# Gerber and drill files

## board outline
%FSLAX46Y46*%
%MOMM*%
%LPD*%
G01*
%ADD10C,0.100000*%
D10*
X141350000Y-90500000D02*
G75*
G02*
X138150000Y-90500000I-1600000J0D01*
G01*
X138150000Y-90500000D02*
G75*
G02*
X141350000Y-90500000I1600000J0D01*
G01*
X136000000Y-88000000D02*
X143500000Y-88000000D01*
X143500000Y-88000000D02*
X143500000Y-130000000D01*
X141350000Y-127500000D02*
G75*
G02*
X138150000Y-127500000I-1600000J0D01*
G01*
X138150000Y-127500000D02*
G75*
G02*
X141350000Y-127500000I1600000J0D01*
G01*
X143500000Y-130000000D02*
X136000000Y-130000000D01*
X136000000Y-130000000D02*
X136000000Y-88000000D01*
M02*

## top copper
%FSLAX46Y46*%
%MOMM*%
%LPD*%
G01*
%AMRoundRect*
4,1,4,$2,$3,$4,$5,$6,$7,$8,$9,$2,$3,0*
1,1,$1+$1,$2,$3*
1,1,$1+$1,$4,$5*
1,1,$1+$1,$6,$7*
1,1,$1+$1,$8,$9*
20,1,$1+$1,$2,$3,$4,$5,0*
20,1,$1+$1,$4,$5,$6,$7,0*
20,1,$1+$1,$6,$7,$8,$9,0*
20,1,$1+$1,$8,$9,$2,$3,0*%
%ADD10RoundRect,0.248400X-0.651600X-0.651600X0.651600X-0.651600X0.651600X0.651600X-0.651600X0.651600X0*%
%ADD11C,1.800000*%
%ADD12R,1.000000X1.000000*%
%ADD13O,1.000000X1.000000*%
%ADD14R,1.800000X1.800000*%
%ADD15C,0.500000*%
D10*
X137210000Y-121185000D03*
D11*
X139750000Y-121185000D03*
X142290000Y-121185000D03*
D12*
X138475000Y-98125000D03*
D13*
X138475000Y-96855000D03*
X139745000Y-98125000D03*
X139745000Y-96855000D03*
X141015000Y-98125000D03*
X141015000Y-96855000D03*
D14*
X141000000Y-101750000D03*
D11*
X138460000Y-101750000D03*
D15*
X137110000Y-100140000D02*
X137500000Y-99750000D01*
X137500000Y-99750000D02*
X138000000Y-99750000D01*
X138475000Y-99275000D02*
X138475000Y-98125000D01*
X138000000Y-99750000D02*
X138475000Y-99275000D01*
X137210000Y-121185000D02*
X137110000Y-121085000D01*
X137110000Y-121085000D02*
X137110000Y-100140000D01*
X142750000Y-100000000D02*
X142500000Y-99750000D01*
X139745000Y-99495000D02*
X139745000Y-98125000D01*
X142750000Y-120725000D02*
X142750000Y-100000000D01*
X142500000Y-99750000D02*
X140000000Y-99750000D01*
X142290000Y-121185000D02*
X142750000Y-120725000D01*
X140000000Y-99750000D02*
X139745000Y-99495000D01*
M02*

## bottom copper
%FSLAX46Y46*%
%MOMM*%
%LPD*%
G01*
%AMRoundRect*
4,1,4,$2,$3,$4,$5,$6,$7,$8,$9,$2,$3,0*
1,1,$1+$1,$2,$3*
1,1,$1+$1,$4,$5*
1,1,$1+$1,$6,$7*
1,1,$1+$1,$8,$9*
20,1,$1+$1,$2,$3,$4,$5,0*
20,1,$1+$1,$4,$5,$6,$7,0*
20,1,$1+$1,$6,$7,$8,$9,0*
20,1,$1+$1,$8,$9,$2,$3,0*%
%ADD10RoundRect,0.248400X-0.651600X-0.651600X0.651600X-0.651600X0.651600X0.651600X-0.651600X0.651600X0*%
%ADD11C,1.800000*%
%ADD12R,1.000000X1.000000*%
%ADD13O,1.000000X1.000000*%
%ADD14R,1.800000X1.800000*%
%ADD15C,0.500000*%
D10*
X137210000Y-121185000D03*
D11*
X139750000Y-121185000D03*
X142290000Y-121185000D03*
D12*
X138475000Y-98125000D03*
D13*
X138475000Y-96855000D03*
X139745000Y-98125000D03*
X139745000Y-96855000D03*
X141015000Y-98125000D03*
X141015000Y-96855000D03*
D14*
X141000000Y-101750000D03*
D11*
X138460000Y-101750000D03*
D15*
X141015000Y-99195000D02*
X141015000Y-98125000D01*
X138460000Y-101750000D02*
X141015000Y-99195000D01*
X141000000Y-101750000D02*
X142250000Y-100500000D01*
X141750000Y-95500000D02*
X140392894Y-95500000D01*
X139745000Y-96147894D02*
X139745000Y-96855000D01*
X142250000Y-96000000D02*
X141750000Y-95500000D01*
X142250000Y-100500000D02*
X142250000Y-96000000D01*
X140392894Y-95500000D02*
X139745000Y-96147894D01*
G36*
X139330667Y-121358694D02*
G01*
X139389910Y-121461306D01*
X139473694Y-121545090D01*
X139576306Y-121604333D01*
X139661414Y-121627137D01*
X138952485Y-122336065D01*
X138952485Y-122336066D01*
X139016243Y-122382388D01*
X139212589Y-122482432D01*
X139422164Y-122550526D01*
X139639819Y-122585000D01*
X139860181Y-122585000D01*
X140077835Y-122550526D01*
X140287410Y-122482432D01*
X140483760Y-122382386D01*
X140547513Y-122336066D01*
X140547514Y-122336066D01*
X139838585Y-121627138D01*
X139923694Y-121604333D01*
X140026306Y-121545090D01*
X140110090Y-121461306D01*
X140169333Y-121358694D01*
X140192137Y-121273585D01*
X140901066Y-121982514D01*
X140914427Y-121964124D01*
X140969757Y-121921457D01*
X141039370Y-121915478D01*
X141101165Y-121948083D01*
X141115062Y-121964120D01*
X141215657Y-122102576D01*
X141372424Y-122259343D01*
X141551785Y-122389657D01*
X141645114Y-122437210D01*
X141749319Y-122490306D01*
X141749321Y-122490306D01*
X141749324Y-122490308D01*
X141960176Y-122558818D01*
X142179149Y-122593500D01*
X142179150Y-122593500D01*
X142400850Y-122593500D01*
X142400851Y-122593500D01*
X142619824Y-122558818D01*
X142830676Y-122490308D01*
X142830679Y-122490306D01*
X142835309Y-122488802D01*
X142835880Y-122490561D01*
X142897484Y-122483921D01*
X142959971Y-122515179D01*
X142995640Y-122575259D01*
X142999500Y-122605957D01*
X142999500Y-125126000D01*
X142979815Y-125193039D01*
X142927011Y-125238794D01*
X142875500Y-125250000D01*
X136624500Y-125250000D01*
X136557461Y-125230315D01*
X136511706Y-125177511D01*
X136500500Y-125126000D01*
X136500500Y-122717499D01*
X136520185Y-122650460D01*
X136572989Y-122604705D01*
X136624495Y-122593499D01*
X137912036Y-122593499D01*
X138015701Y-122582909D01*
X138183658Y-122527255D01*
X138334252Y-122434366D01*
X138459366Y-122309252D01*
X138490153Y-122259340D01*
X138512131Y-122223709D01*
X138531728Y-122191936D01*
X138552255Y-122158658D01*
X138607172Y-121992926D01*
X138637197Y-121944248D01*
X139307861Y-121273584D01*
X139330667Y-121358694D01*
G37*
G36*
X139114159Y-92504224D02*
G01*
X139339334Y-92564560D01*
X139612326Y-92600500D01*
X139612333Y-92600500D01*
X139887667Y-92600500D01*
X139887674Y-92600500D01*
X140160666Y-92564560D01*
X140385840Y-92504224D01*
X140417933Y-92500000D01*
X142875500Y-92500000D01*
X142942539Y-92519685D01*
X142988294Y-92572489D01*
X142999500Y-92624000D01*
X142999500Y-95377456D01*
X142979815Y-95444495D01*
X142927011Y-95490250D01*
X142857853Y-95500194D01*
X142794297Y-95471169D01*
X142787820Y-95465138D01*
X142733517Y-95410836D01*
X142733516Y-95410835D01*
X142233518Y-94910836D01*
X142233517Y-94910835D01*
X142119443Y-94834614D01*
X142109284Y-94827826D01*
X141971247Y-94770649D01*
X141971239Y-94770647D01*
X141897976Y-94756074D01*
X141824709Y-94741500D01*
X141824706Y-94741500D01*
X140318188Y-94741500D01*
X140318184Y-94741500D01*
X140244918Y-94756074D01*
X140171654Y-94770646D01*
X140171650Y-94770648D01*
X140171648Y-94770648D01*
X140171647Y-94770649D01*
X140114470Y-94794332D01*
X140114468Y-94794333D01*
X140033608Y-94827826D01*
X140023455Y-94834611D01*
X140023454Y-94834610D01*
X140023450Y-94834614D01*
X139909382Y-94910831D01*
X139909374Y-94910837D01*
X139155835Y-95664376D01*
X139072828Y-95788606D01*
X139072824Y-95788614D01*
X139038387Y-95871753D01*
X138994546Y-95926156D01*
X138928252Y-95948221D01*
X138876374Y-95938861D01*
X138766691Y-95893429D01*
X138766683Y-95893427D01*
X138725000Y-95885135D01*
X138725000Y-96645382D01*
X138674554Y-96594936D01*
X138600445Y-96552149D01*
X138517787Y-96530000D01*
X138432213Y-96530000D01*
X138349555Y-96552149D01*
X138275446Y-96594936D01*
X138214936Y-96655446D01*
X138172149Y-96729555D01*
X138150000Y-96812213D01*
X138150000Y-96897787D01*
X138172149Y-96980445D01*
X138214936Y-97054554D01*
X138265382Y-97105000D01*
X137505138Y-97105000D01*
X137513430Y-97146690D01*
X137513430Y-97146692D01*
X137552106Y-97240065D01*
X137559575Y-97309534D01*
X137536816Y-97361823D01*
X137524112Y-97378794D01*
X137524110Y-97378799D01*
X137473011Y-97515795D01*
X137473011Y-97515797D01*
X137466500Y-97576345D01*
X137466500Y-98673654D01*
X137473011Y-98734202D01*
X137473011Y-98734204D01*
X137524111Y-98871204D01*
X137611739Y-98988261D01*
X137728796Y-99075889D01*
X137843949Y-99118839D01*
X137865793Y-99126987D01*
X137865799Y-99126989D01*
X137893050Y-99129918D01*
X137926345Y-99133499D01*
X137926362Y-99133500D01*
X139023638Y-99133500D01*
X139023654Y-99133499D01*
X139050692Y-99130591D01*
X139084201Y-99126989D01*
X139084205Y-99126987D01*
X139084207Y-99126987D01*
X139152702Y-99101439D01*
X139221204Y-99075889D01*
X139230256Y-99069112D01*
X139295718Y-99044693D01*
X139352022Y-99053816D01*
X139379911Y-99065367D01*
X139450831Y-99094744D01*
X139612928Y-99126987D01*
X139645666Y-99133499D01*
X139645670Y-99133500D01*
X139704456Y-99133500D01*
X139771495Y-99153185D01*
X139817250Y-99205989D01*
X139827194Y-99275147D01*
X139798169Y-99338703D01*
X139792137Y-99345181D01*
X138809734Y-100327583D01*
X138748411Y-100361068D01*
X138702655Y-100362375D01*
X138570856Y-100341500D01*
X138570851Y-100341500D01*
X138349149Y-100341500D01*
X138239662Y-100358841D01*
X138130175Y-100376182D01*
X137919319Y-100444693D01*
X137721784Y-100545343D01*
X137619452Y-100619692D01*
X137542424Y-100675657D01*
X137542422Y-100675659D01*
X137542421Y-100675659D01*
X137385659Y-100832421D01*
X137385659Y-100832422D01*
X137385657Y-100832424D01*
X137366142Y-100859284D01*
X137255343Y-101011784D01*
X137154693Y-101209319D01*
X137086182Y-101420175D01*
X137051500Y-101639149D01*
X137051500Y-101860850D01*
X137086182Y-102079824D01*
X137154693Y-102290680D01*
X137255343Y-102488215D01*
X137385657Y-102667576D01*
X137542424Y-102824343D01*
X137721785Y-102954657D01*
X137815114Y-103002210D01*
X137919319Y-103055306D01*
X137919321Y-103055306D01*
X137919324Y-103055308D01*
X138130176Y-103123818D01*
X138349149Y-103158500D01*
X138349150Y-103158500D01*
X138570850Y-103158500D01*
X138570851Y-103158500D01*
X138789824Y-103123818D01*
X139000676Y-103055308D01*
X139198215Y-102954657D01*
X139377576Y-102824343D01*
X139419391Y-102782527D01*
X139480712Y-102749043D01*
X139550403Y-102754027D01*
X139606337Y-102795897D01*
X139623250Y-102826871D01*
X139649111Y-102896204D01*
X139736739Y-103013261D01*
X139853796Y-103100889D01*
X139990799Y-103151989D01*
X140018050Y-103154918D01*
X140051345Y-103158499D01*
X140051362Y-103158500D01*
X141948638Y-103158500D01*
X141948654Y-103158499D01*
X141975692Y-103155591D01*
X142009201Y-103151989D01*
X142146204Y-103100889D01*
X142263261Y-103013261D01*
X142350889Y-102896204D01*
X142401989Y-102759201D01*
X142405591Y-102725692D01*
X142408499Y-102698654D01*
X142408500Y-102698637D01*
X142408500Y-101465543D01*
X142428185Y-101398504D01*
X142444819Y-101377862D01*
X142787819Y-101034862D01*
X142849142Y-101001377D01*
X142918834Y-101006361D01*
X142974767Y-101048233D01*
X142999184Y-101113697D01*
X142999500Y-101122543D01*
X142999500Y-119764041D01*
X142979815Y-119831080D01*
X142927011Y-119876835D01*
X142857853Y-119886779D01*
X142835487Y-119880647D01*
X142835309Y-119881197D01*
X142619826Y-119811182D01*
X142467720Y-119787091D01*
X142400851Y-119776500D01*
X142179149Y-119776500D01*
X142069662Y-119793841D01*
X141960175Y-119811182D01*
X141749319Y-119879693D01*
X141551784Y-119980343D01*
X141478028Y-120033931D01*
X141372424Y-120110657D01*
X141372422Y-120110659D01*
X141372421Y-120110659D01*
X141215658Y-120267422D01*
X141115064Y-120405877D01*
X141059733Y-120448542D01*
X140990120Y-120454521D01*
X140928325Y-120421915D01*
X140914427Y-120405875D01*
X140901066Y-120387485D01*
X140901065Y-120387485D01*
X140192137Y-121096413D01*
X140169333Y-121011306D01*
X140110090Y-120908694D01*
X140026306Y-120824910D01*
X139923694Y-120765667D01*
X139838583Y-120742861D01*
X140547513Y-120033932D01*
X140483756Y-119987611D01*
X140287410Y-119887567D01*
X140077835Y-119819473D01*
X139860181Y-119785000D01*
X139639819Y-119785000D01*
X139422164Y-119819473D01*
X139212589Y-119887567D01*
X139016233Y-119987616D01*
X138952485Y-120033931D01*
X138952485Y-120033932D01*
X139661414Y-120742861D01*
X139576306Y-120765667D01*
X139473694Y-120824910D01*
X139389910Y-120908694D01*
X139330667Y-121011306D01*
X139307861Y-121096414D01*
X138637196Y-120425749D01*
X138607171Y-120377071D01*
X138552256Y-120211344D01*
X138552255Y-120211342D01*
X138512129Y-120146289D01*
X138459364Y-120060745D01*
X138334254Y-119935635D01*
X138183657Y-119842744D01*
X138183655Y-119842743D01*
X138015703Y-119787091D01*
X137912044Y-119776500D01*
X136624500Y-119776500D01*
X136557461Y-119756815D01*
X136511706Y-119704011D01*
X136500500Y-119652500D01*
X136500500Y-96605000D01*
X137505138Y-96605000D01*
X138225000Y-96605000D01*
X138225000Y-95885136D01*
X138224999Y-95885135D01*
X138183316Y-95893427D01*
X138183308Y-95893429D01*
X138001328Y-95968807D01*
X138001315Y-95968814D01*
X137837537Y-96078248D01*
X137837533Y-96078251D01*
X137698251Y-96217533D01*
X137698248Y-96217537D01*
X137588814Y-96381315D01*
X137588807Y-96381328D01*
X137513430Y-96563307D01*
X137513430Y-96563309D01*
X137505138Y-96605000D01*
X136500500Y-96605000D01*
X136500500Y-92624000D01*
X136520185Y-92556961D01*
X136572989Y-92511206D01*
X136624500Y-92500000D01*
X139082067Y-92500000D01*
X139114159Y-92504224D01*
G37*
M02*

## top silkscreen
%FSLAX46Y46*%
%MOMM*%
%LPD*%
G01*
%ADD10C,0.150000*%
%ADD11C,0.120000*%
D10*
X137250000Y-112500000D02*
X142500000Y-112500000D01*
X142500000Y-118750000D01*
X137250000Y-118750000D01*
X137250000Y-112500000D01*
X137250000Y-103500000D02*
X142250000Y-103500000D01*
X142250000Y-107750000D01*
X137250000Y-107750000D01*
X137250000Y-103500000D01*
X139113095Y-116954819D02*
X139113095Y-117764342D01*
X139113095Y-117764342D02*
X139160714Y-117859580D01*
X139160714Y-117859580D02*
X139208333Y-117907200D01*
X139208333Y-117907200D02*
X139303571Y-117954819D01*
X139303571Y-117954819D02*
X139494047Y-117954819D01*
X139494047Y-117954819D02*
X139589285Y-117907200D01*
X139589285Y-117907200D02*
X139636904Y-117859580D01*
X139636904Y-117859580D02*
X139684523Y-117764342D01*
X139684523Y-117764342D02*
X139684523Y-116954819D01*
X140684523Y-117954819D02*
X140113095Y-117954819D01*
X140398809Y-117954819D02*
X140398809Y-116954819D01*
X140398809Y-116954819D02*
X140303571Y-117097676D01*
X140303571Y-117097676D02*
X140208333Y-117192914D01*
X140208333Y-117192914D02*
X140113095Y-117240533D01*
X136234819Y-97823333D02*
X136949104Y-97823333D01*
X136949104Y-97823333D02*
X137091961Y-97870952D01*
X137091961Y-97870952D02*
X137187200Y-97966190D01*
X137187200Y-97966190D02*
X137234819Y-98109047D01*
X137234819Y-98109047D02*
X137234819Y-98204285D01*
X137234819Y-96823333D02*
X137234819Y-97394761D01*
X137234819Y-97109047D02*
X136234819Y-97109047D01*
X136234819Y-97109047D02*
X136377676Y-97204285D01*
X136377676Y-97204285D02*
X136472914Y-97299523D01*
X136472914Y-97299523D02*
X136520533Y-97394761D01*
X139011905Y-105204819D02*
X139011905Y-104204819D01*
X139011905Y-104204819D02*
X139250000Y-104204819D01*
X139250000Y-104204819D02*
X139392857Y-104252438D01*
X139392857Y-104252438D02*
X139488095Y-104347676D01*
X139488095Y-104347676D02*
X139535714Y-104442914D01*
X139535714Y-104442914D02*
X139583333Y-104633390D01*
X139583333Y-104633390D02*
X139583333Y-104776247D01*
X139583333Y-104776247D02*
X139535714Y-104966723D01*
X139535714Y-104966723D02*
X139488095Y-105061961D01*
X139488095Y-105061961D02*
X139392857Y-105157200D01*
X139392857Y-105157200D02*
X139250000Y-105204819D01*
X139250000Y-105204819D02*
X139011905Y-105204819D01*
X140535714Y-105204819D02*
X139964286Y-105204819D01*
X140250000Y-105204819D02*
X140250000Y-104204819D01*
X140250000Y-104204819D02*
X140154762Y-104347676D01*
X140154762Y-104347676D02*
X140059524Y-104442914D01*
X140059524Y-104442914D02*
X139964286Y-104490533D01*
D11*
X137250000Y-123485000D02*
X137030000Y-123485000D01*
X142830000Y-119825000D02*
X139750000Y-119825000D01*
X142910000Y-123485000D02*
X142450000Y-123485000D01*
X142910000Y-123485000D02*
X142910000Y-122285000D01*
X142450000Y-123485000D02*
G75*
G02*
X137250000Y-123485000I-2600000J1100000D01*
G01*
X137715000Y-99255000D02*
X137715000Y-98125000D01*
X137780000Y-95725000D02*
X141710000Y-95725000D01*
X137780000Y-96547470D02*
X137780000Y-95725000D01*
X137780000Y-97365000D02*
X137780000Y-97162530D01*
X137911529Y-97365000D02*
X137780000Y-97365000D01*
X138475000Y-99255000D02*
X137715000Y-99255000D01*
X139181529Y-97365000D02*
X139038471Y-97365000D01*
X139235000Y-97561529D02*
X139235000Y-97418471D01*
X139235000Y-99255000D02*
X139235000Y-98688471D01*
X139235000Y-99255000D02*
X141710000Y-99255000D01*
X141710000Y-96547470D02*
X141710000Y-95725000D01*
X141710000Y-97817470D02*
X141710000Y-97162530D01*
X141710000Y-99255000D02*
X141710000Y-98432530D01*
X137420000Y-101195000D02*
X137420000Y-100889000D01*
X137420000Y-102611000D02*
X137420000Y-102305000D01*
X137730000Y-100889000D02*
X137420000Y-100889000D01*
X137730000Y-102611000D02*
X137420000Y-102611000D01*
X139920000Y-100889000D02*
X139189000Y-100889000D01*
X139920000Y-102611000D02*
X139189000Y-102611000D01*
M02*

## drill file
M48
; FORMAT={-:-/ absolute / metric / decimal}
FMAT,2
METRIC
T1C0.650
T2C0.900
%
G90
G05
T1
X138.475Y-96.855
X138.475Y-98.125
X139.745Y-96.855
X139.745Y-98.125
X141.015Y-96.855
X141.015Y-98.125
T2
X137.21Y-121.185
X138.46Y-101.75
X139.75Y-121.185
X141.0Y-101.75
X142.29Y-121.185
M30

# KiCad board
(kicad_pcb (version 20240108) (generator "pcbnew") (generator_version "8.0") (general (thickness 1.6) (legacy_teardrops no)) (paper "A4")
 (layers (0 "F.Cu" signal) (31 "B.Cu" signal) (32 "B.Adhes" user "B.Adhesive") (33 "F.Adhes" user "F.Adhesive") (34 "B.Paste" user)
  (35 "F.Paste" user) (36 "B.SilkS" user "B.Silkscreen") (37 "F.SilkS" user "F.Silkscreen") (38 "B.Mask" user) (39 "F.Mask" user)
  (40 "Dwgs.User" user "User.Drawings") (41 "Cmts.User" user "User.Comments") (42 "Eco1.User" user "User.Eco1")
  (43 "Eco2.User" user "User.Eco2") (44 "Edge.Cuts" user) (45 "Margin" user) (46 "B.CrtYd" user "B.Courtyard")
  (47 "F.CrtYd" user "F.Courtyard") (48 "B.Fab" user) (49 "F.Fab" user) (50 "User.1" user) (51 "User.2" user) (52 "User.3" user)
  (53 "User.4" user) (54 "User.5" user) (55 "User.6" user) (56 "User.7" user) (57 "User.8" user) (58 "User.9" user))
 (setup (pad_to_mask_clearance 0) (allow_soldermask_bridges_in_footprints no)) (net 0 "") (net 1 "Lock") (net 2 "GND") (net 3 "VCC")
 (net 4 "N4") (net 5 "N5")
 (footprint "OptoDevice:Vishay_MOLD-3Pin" (layer "F.Cu") (at 137.21 121.185)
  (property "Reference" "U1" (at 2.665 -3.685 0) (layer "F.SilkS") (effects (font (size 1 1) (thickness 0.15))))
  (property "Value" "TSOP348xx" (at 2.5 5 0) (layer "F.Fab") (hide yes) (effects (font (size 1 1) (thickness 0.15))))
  (fp_line (start 0.04 2.3) (end -0.18 2.3) (stroke (width 0.12) (type solid)) (layer "F.SilkS"))
  (fp_line (start 5.62 -1.36) (end 2.54 -1.36) (stroke (width 0.12) (type solid)) (layer "F.SilkS"))
  (fp_line (start 5.7 2.3) (end 5.24 2.3) (stroke (width 0.12) (type solid)) (layer "F.SilkS"))
  (fp_line (start 5.7 2.3) (end 5.7 1.1) (stroke (width 0.12) (type solid)) (layer "F.SilkS"))
  (fp_arc (start 5.24 2.3) (mid 2.64 4.023119) (end 0.04 2.3) (stroke (width 0.12) (type solid)) (layer "F.SilkS"))
  (pad "1" thru_hole roundrect (at 0 0) (size 1.8 1.8) (drill 0.9) (layers "*.Cu" "*.Mask") (remove_unused_layers no)
   (roundrect_rratio 0.138) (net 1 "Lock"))
  (pad "2" thru_hole circle (at 2.54 0) (size 1.8 1.8) (drill 0.9) (layers "*.Cu" "*.Mask") (remove_unused_layers no) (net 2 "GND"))
  (pad "3" thru_hole circle (at 5.08 0) (size 1.8 1.8) (drill 0.9) (layers "*.Cu" "*.Mask") (remove_unused_layers no) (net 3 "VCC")))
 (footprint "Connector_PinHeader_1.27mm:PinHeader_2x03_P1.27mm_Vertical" (layer "F.Cu") (at 138.475 98.125 90)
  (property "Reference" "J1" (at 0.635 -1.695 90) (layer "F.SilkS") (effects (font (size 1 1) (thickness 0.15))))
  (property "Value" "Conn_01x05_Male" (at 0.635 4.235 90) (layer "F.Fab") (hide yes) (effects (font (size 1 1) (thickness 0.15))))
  (fp_line (start -1.13 -0.76) (end 0 -0.76) (stroke (width 0.12) (type solid)) (layer "F.SilkS"))
  (fp_line (start 2.4 -0.695) (end 2.4 3.235) (stroke (width 0.12) (type solid)) (layer "F.SilkS"))
  (fp_line (start 1.57753 -0.695) (end 2.4 -0.695) (stroke (width 0.12) (type solid)) (layer "F.SilkS"))
  (fp_line (start 0.76 -0.695) (end 0.96247 -0.695) (stroke (width 0.12) (type solid)) (layer "F.SilkS"))
  (fp_line (start 0.76 -0.563471) (end 0.76 -0.695) (stroke (width 0.12) (type solid)) (layer "F.SilkS"))
  (fp_line (start -1.13 0) (end -1.13 -0.76) (stroke (width 0.12) (type solid)) (layer "F.SilkS"))
  (fp_line (start 0.76 0.706529) (end 0.76 0.563471) (stroke (width 0.12) (type solid)) (layer "F.SilkS"))
  (fp_line (start 0.563471 0.76) (end 0.706529 0.76) (stroke (width 0.12) (type solid)) (layer "F.SilkS"))
  (fp_line (start -1.13 0.76) (end -0.563471 0.76) (stroke (width 0.12) (type solid)) (layer "F.SilkS"))
  (fp_line (start -1.13 0.76) (end -1.13 3.235) (stroke (width 0.12) (type solid)) (layer "F.SilkS"))
  (fp_line (start 1.57753 3.235) (end 2.4 3.235) (stroke (width 0.12) (type solid)) (layer "F.SilkS"))
  (fp_line (start 0.30753 3.235) (end 0.96247 3.235) (stroke (width 0.12) (type solid)) (layer "F.SilkS"))
  (fp_line (start -1.13 3.235) (end -0.30753 3.235) (stroke (width 0.12) (type solid)) (layer "F.SilkS"))
  (pad "1" thru_hole rect (at 0 0 90) (size 1 1) (drill 0.65) (layers "*.Cu" "*.Mask") (remove_unused_layers no) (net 1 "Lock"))
  (pad "2" thru_hole oval (at 1.27 0 90) (size 1 1) (drill 0.65) (layers "*.Cu" "*.Mask") (remove_unused_layers no) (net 2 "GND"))
  (pad "3" thru_hole oval (at 0 1.27 90) (size 1 1) (drill 0.65) (layers "*.Cu" "*.Mask") (remove_unused_layers no) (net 3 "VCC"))
  (pad "4" thru_hole oval (at 1.27 1.27 90) (size 1 1) (drill 0.65) (layers "*.Cu" "*.Mask") (remove_unused_layers no) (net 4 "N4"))
  (pad "5" thru_hole oval (at 0 2.54 90) (size 1 1) (drill 0.65) (layers "*.Cu" "*.Mask") (remove_unused_layers no) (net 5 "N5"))
  (pad "6" thru_hole oval (at 1.27 2.54 90) (size 1 1) (drill 0.65) (layers "*.Cu" "*.Mask") (remove_unused_layers no)))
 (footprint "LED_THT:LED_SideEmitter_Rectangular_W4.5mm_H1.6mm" (layer "F.Cu") (at 141 101.75 180)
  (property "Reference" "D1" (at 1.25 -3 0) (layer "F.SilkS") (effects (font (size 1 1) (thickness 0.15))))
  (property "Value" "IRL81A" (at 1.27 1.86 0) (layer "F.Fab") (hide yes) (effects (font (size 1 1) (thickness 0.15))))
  (fp_line (start 3.58 0.555) (end 3.58 0.861) (stroke (width 0.12) (type solid)) (layer "F.SilkS"))
  (fp_line (start 3.58 -0.861) (end 3.58 -0.555) (stroke (width 0.12) (type solid)) (layer "F.SilkS"))
  (fp_line (start 3.27 0.861) (end 3.58 0.861) (stroke (width 0.12) (type solid)) (layer "F.SilkS"))
  (fp_line (start 3.27 -0.861) (end 3.58 -0.861) (stroke (width 0.12) (type solid)) (layer "F.SilkS"))
  (fp_line (start 1.08 0.861) (end 1.811 0.861) (stroke (width 0.12) (type solid)) (layer "F.SilkS"))
  (fp_line (start 1.08 -0.861) (end 1.811 -0.861) (stroke (width 0.12) (type solid)) (layer "F.SilkS"))
  (pad "1" thru_hole rect (at 0 0 180) (size 1.8 1.8) (drill 0.9) (layers "*.Cu" "*.Mask") (remove_unused_layers no) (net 4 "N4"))
  (pad "2" thru_hole circle (at 2.54 0 180) (size 1.8 1.8) (drill 0.9) (layers "*.Cu" "*.Mask") (remove_unused_layers no) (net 5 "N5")))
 (gr_rect (start 137.25 112.5) (end 142.5 118.75) (stroke (width 0.15) (type default)) (fill none) (layer "F.SilkS"))
 (gr_rect (start 137.25 103.5) (end 142.25 107.75) (stroke (width 0.15) (type default)) (fill none) (layer "F.SilkS"))
 (gr_circle (center 139.75 90.5) (end 141.35 90.5) (stroke (width 0.1) (type default)) (fill none) (layer "Edge.Cuts"))
 (gr_line (start 136 88) (end 143.5 88) (stroke (width 0.1) (type solid)) (layer "Edge.Cuts"))
 (gr_line (start 143.5 88) (end 143.5 130) (stroke (width 0.1) (type solid)) (layer "Edge.Cuts"))
 (gr_circle (center 139.75 127.5) (end 141.35 127.5) (stroke (width 0.1) (type default)) (fill none) (layer "Edge.Cuts"))
 (gr_line (start 143.5 130) (end 136 130) (stroke (width 0.1) (type solid)) (layer "Edge.Cuts"))
 (gr_line (start 136 130) (end 136 88) (stroke (width 0.1) (type solid)) (layer "Edge.Cuts"))
 (segment (start 141.015 99.195) (end 141.015 98.125) (width 0.5) (layer "B.Cu") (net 5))
 (segment (start 138.46 101.75) (end 141.015 99.195) (width 0.5) (layer "B.Cu") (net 5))
 (segment (start 141 101.75) (end 142.25 100.5) (width 0.5) (layer "B.Cu") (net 4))
 (segment (start 141.75 95.5) (end 140.392894 95.5) (width 0.5) (layer "B.Cu") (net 4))
 (segment (start 139.745 96.147894) (end 139.745 96.855) (width 0.5) (layer "B.Cu") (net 4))
 (segment (start 142.25 96) (end 141.75 95.5) (width 0.5) (layer "B.Cu") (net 4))
 (segment (start 142.25 100.5) (end 142.25 96) (width 0.5) (layer "B.Cu") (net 4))
 (segment (start 140.392894 95.5) (end 139.745 96.147894) (width 0.5) (layer "B.Cu") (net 4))
 (segment (start 137.11 100.14) (end 137.5 99.75) (width 0.5) (layer "F.Cu") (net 1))
 (segment (start 137.5 99.75) (end 138 99.75) (width 0.5) (layer "F.Cu") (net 1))
 (segment (start 138.475 99.275) (end 138.475 98.125) (width 0.5) (layer "F.Cu") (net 1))
 (segment (start 138 99.75) (end 138.475 99.275) (width 0.5) (layer "F.Cu") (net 1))
 (segment (start 137.21 121.185) (end 137.11 121.085) (width 0.5) (layer "F.Cu") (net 1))
 (segment (start 137.11 121.085) (end 137.11 100.14) (width 0.5) (layer "F.Cu") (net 1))
 (segment (start 142.75 100) (end 142.5 99.75) (width 0.5) (layer "F.Cu") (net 3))
 (segment (start 139.745 99.495) (end 139.745 98.125) (width 0.5) (layer "F.Cu") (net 3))
 (segment (start 142.75 120.725) (end 142.75 100) (width 0.5) (layer "F.Cu") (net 3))
 (segment (start 142.5 99.75) (end 140 99.75) (width 0.5) (layer "F.Cu") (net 3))
 (segment (start 142.29 121.185) (end 142.75 120.725) (width 0.5) (layer "F.Cu") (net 3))
 (segment (start 140 99.75) (end 139.745 99.495) (width 0.5) (layer "F.Cu") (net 3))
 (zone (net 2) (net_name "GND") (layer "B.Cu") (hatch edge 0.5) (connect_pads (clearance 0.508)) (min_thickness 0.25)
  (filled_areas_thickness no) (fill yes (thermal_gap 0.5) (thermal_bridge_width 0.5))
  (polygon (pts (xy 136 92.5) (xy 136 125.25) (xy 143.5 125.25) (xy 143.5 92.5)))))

